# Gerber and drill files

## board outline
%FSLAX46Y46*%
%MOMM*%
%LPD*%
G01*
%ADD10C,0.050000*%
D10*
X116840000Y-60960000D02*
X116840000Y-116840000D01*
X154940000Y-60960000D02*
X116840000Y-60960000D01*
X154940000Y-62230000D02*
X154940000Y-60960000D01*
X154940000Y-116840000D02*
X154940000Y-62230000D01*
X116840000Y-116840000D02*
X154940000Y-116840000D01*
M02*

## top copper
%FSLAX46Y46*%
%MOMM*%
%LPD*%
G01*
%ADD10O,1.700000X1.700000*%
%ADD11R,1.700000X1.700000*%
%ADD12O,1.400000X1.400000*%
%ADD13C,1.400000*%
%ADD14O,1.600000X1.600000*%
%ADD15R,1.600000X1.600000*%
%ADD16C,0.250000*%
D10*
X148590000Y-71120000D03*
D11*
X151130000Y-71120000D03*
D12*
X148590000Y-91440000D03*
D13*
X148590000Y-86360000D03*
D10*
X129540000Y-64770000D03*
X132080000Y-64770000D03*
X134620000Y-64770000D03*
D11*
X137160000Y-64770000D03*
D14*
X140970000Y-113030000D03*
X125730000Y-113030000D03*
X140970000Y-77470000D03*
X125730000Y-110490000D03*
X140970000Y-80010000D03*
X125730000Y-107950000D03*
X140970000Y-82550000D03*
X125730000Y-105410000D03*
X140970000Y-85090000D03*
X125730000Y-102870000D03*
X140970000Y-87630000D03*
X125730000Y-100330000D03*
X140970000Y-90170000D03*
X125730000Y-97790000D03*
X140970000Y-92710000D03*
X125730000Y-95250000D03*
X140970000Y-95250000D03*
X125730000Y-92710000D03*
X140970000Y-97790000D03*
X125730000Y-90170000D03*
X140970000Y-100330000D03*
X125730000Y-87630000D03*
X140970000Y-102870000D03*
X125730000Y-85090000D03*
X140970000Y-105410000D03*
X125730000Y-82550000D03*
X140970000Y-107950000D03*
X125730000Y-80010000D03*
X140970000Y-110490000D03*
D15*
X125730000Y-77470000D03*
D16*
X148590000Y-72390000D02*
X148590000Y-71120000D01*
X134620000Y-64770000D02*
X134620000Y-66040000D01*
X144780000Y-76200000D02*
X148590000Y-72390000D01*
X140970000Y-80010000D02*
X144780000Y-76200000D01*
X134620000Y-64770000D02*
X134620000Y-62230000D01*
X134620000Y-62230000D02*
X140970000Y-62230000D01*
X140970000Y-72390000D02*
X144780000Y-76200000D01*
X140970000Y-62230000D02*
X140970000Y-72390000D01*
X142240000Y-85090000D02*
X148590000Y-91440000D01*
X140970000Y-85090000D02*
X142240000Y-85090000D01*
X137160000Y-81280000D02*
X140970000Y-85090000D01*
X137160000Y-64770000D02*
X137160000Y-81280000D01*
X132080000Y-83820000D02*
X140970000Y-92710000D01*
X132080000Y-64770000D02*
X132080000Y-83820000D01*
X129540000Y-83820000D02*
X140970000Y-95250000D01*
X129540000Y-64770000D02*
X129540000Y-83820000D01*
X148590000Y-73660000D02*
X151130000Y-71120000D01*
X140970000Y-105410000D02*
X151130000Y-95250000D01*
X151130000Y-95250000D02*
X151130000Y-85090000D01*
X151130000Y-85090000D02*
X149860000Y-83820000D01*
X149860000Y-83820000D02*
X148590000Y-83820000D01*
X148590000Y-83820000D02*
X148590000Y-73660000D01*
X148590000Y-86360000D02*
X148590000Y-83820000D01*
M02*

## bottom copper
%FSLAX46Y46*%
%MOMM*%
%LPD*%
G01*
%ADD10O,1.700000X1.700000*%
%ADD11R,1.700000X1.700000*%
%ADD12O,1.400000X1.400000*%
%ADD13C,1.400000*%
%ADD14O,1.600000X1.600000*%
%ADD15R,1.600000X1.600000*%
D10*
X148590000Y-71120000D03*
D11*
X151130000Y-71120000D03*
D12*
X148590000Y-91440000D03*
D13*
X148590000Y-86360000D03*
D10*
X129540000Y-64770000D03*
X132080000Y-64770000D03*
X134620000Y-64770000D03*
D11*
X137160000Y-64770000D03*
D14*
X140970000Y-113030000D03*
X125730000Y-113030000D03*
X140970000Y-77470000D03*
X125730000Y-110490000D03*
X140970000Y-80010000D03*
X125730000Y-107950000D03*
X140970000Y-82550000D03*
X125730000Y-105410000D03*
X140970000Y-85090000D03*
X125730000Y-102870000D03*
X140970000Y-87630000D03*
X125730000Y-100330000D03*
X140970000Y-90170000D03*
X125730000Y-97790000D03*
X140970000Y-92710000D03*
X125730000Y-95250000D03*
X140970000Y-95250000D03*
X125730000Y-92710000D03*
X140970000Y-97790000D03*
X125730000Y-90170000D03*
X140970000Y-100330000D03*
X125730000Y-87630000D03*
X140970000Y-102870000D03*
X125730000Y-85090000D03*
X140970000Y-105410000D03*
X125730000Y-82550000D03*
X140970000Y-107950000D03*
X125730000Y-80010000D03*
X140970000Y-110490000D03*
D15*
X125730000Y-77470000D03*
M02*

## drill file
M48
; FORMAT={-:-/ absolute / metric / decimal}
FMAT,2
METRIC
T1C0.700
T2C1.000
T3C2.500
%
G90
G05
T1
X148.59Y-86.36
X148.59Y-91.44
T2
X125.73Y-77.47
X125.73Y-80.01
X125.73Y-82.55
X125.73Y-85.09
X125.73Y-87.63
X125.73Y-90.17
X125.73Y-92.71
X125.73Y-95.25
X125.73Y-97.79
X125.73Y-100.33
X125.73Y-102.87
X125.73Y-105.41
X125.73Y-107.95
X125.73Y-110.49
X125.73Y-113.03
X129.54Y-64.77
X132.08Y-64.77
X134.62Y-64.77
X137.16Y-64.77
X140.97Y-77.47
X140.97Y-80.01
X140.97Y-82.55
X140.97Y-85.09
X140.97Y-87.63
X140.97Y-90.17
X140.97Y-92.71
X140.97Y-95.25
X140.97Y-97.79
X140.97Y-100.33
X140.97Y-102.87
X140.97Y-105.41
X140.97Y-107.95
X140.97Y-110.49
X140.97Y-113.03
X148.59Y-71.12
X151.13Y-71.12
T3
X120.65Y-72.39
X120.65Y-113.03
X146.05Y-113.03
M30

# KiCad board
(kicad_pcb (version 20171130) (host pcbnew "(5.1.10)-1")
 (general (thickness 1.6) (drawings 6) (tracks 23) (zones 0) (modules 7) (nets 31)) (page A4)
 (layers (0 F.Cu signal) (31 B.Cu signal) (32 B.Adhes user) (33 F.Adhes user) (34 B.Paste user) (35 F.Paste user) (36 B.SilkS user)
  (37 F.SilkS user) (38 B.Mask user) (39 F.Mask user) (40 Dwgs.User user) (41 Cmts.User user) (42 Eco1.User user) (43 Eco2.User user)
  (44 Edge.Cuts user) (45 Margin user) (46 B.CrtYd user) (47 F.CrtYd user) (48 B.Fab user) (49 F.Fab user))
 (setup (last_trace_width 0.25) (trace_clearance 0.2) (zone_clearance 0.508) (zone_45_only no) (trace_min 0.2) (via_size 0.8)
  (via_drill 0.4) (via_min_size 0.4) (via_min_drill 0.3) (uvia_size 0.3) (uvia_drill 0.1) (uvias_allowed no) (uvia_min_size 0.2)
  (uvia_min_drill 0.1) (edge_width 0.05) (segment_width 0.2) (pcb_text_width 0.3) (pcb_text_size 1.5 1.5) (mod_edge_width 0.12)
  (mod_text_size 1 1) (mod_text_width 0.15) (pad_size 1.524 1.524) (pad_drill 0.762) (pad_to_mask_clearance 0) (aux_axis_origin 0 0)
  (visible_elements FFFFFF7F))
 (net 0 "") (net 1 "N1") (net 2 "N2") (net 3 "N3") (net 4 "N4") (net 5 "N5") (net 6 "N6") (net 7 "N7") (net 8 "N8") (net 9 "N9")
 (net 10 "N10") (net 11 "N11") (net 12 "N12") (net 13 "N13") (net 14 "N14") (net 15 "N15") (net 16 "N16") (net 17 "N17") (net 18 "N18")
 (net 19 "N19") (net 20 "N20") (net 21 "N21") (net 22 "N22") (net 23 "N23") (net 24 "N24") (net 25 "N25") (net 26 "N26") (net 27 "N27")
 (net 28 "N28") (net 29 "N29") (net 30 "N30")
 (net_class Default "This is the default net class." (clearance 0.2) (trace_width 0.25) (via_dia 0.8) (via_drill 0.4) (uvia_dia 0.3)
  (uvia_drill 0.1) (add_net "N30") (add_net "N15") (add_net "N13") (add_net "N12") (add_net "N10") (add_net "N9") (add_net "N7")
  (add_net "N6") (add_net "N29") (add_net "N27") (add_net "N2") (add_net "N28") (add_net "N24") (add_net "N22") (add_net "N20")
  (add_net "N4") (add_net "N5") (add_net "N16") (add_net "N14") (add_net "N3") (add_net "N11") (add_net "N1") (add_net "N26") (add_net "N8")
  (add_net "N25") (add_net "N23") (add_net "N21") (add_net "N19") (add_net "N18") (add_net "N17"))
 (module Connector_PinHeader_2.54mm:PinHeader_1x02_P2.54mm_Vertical (layer F.Cu) (at 151.13 71.12 270)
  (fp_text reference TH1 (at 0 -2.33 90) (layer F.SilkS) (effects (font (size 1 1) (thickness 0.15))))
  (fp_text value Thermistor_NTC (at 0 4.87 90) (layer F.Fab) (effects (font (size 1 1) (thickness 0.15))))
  (pad 2 thru_hole oval (at 0 2.54 270) (size 1.7 1.7) (drill 1) (layers *.Cu *.Mask) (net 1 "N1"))
  (pad 1 thru_hole rect (at 0 0 270) (size 1.7 1.7) (drill 1) (layers *.Cu *.Mask) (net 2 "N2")))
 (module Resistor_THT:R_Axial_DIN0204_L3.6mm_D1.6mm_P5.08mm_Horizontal (layer F.Cu) (at 148.59 86.36 270)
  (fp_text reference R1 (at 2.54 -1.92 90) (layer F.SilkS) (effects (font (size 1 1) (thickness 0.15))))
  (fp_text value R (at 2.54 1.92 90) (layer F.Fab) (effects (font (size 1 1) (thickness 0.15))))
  (pad 2 thru_hole oval (at 5.08 0 270) (size 1.4 1.4) (drill 0.7) (layers *.Cu *.Mask) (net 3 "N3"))
  (pad 1 thru_hole circle (at 0 0 270) (size 1.4 1.4) (drill 0.7) (layers *.Cu *.Mask) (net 2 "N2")))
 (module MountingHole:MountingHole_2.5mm (layer F.Cu) (at 146.05 113.03)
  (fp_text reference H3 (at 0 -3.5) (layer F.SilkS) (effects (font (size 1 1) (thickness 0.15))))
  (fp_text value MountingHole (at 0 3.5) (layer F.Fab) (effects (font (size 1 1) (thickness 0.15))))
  (pad 1 np_thru_hole circle (at 0 0) (size 2.5 2.5) (drill 2.5) (layers *.Cu *.Mask)))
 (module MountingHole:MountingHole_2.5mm (layer F.Cu) (at 120.65 113.03)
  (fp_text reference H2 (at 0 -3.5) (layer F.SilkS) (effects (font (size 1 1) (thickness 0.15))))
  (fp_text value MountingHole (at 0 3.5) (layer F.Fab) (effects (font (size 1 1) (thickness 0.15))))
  (pad 1 np_thru_hole circle (at 0 0) (size 2.5 2.5) (drill 2.5) (layers *.Cu *.Mask)))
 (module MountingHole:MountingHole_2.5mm (layer F.Cu) (at 120.65 72.39)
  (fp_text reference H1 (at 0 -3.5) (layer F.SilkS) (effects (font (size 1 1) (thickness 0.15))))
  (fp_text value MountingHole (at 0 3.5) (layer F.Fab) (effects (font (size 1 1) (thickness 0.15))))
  (pad 1 np_thru_hole circle (at 0 0) (size 2.5 2.5) (drill 2.5) (layers *.Cu *.Mask)))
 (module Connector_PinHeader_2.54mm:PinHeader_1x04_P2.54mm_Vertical (layer F.Cu) (at 137.16 64.77 270)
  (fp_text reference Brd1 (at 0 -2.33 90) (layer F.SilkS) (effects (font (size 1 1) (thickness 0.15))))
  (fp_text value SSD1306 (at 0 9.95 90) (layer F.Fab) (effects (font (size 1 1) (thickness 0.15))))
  (pad 4 thru_hole oval (at 0 7.62 270) (size 1.7 1.7) (drill 1) (layers *.Cu *.Mask) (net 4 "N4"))
  (pad 3 thru_hole oval (at 0 5.08 270) (size 1.7 1.7) (drill 1) (layers *.Cu *.Mask) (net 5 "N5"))
  (pad 2 thru_hole oval (at 0 2.54 270) (size 1.7 1.7) (drill 1) (layers *.Cu *.Mask) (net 1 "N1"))
  (pad 1 thru_hole rect (at 0 0 270) (size 1.7 1.7) (drill 1) (layers *.Cu *.Mask) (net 3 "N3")))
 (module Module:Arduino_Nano (layer F.Cu) (at 125.73 77.47)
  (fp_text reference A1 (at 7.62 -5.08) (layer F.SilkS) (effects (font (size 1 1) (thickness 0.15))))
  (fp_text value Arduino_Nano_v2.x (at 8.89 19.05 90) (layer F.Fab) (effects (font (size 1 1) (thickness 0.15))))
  (pad 16 thru_hole oval (at 15.24 35.56) (size 1.6 1.6) (drill 1) (layers *.Cu *.Mask) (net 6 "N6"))
  (pad 15 thru_hole oval (at 0 35.56) (size 1.6 1.6) (drill 1) (layers *.Cu *.Mask) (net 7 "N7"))
  (pad 30 thru_hole oval (at 15.24 0) (size 1.6 1.6) (drill 1) (layers *.Cu *.Mask) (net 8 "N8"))
  (pad 14 thru_hole oval (at 0 33.02) (size 1.6 1.6) (drill 1) (layers *.Cu *.Mask) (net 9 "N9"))
  (pad 29 thru_hole oval (at 15.24 2.54) (size 1.6 1.6) (drill 1) (layers *.Cu *.Mask) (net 1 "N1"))
  (pad 13 thru_hole oval (at 0 30.48) (size 1.6 1.6) (drill 1) (layers *.Cu *.Mask) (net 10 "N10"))
  (pad 28 thru_hole oval (at 15.24 5.08) (size 1.6 1.6) (drill 1) (layers *.Cu *.Mask) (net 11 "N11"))
  (pad 12 thru_hole oval (at 0 27.94) (size 1.6 1.6) (drill 1) (layers *.Cu *.Mask) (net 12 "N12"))
  (pad 27 thru_hole oval (at 15.24 7.62) (size 1.6 1.6) (drill 1) (layers *.Cu *.Mask) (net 3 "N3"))
  (pad 11 thru_hole oval (at 0 25.4) (size 1.6 1.6) (drill 1) (layers *.Cu *.Mask) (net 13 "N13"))
  (pad 26 thru_hole oval (at 15.24 10.16) (size 1.6 1.6) (drill 1) (layers *.Cu *.Mask) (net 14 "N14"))
  (pad 10 thru_hole oval (at 0 22.86) (size 1.6 1.6) (drill 1) (layers *.Cu *.Mask) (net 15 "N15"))
  (pad 25 thru_hole oval (at 15.24 12.7) (size 1.6 1.6) (drill 1) (layers *.Cu *.Mask) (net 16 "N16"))
  (pad 9 thru_hole oval (at 0 20.32) (size 1.6 1.6) (drill 1) (layers *.Cu *.Mask) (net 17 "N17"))
  (pad 24 thru_hole oval (at 15.24 15.24) (size 1.6 1.6) (drill 1) (layers *.Cu *.Mask) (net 5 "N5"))
  (pad 8 thru_hole oval (at 0 17.78) (size 1.6 1.6) (drill 1) (layers *.Cu *.Mask) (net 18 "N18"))
  (pad 23 thru_hole oval (at 15.24 17.78) (size 1.6 1.6) (drill 1) (layers *.Cu *.Mask) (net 4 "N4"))
  (pad 7 thru_hole oval (at 0 15.24) (size 1.6 1.6) (drill 1) (layers *.Cu *.Mask) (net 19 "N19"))
  (pad 22 thru_hole oval (at 15.24 20.32) (size 1.6 1.6) (drill 1) (layers *.Cu *.Mask) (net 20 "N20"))
  (pad 6 thru_hole oval (at 0 12.7) (size 1.6 1.6) (drill 1) (layers *.Cu *.Mask) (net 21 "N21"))
  (pad 21 thru_hole oval (at 15.24 22.86) (size 1.6 1.6) (drill 1) (layers *.Cu *.Mask) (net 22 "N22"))
  (pad 5 thru_hole oval (at 0 10.16) (size 1.6 1.6) (drill 1) (layers *.Cu *.Mask) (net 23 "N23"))
  (pad 20 thru_hole oval (at 15.24 25.4) (size 1.6 1.6) (drill 1) (layers *.Cu *.Mask) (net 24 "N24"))
  (pad 4 thru_hole oval (at 0 7.62) (size 1.6 1.6) (drill 1) (layers *.Cu *.Mask) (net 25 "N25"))
  (pad 19 thru_hole oval (at 15.24 27.94) (size 1.6 1.6) (drill 1) (layers *.Cu *.Mask) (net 2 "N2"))
  (pad 3 thru_hole oval (at 0 5.08) (size 1.6 1.6) (drill 1) (layers *.Cu *.Mask) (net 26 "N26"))
  (pad 18 thru_hole oval (at 15.24 30.48) (size 1.6 1.6) (drill 1) (layers *.Cu *.Mask) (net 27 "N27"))
  (pad 2 thru_hole oval (at 0 2.54) (size 1.6 1.6) (drill 1) (layers *.Cu *.Mask) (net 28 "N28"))
  (pad 17 thru_hole oval (at 15.24 33.02) (size 1.6 1.6) (drill 1) (layers *.Cu *.Mask) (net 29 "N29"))
  (pad 1 thru_hole rect (at 0 0) (size 1.6 1.6) (drill 1) (layers *.Cu *.Mask) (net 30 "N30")))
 (gr_line (start 116.84 60.96) (end 116.84 116.84) (layer Edge.Cuts) (width 0.05))
 (gr_line (start 154.94 60.96) (end 116.84 60.96) (layer Edge.Cuts) (width 0.05))
 (gr_line (start 154.94 62.23) (end 154.94 60.96) (layer Edge.Cuts) (width 0.05))
 (gr_line (start 154.94 116.84) (end 154.94 62.23) (layer Edge.Cuts) (width 0.05))
 (gr_line (start 116.84 116.84) (end 154.94 116.84) (layer Edge.Cuts) (width 0.05))
 (segment (start 148.59 72.39) (end 148.59 71.12) (width 0.25) (layer F.Cu) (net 1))
 (segment (start 134.62 64.77) (end 134.62 66.04) (width 0.25) (layer F.Cu) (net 1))
 (segment (start 144.78 76.2) (end 148.59 72.39) (width 0.25) (layer F.Cu) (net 1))
 (segment (start 140.97 80.01) (end 144.78 76.2) (width 0.25) (layer F.Cu) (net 1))
 (segment (start 134.62 64.77) (end 134.62 62.23) (width 0.25) (layer F.Cu) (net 1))
 (segment (start 134.62 62.23) (end 140.97 62.23) (width 0.25) (layer F.Cu) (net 1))
 (segment (start 140.97 72.39) (end 144.78 76.2) (width 0.25) (layer F.Cu) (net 1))
 (segment (start 140.97 62.23) (end 140.97 72.39) (width 0.25) (layer F.Cu) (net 1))
 (segment (start 142.24 85.09) (end 148.59 91.44) (width 0.25) (layer F.Cu) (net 3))
 (segment (start 140.97 85.09) (end 142.24 85.09) (width 0.25) (layer F.Cu) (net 3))
 (segment (start 137.16 81.28) (end 140.97 85.09) (width 0.25) (layer F.Cu) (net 3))
 (segment (start 137.16 64.77) (end 137.16 81.28) (width 0.25) (layer F.Cu) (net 3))
 (segment (start 132.08 83.82) (end 140.97 92.71) (width 0.25) (layer F.Cu) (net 5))
 (segment (start 132.08 64.77) (end 132.08 83.82) (width 0.25) (layer F.Cu) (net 5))
 (segment (start 129.54 83.82) (end 140.97 95.25) (width 0.25) (layer F.Cu) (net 4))
 (segment (start 129.54 64.77) (end 129.54 83.82) (width 0.25) (layer F.Cu) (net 4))
 (segment (start 148.59 73.66) (end 151.13 71.12) (width 0.25) (layer F.Cu) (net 2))
 (segment (start 140.97 105.41) (end 151.13 95.25) (width 0.25) (layer F.Cu) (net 2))
 (segment (start 151.13 95.25) (end 151.13 85.09) (width 0.25) (layer F.Cu) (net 2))
 (segment (start 151.13 85.09) (end 149.86 83.82) (width 0.25) (layer F.Cu) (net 2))
 (segment (start 149.86 83.82) (end 148.59 83.82) (width 0.25) (layer F.Cu) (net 2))
 (segment (start 148.59 83.82) (end 148.59 73.66) (width 0.25) (layer F.Cu) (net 2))
 (segment (start 148.59 86.36) (end 148.59 83.82) (width 0.25) (layer F.Cu) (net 2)))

